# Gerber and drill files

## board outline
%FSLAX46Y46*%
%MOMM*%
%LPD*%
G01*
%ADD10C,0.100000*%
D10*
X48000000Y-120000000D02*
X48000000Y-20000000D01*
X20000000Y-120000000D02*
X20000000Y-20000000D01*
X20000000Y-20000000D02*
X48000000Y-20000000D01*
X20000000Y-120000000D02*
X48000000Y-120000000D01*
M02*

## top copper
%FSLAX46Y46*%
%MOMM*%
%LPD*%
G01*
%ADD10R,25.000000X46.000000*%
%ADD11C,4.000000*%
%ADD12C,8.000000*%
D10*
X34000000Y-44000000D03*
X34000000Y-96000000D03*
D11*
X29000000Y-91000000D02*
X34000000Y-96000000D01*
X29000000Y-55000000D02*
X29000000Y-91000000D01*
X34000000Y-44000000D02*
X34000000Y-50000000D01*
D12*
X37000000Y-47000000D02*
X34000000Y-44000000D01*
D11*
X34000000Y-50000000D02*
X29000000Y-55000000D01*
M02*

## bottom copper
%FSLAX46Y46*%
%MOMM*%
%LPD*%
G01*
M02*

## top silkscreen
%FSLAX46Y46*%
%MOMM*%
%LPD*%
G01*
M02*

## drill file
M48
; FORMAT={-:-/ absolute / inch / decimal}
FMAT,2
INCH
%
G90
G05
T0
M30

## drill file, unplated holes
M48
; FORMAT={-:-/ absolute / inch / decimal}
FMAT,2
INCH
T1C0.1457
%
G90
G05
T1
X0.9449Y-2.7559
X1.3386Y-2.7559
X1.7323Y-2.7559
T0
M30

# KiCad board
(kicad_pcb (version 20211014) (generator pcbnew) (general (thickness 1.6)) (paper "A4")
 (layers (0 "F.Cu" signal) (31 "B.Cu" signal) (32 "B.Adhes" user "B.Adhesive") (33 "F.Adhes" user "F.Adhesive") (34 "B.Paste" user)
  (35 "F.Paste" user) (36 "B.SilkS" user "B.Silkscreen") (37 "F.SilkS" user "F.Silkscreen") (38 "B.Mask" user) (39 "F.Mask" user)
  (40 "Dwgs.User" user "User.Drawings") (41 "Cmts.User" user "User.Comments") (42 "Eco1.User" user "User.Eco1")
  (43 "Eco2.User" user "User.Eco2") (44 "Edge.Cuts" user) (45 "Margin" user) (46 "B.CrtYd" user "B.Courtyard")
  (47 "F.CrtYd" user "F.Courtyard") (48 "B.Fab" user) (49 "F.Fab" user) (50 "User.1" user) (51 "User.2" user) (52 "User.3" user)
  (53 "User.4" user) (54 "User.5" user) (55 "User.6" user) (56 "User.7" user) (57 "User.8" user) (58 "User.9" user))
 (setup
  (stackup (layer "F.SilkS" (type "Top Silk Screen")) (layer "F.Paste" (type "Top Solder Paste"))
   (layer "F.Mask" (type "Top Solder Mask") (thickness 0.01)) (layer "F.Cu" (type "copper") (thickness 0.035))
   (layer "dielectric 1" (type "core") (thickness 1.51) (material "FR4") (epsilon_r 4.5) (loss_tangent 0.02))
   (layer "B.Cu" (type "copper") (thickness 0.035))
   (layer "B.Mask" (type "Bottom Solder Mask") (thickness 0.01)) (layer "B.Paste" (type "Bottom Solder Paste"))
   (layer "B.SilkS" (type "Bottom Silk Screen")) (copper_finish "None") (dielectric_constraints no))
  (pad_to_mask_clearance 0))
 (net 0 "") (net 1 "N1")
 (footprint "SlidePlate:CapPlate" (layer "F.Cu") (at 34 44)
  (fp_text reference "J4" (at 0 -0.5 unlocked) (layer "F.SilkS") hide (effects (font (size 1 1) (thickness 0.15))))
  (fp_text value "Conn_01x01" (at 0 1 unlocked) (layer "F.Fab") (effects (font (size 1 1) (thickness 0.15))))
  (pad "1" smd rect (at 0 0) (size 25 46) (layers "F.Cu") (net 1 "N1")))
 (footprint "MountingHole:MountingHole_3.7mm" (layer "F.Cu") (at 24 70)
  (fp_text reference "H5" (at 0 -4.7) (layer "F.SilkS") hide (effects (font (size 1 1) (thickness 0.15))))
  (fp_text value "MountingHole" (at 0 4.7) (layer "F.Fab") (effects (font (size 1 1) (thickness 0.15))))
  (pad "" np_thru_hole circle (at 0 0) (size 3.7 3.7) (drill 3.7) (layers *.Cu *.Mask)))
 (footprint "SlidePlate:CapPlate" (layer "F.Cu") (at 34 96)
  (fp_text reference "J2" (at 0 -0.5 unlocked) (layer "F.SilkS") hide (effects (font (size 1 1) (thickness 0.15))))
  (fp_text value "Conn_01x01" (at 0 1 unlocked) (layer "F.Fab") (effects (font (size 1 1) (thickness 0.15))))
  (pad "1" smd rect (at 0 0) (size 25 46) (layers "F.Cu") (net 1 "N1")))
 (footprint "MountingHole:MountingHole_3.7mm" (layer "F.Cu") (at 34 70)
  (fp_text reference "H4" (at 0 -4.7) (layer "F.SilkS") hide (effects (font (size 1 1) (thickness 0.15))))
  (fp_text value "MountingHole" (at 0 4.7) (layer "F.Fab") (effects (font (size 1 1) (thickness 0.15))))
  (pad "" np_thru_hole circle (at 0 0) (size 3.7 3.7) (drill 3.7) (layers *.Cu *.Mask)))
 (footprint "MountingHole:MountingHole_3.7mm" (layer "F.Cu") (at 44 70)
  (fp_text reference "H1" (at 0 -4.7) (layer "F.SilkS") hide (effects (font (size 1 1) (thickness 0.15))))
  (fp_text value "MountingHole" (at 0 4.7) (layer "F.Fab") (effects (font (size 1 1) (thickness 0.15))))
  (pad "" np_thru_hole circle (at 0 0) (size 3.7 3.7) (drill 3.7) (layers *.Cu *.Mask)))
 (gr_line (start 48 120) (end 48 20) (layer "Edge.Cuts") (width 0.1))
 (gr_line (start 20 120) (end 20 20) (layer "Edge.Cuts") (width 0.1))
 (gr_line (start 20 20) (end 48 20) (layer "Edge.Cuts") (width 0.1))
 (gr_line (start 20 120) (end 48 120) (layer "Edge.Cuts") (width 0.1))
 (segment (start 29 91) (end 34 96) (width 4) (layer "F.Cu") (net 1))
 (segment (start 29 55) (end 29 91) (width 4) (layer "F.Cu") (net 1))
 (segment (start 34 44) (end 34 50) (width 4) (layer "F.Cu") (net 1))
 (segment (start 37 47) (end 34 44) (width 8) (layer "F.Cu") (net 1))
 (segment (start 34 50) (end 29 55) (width 4) (layer "F.Cu") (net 1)))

